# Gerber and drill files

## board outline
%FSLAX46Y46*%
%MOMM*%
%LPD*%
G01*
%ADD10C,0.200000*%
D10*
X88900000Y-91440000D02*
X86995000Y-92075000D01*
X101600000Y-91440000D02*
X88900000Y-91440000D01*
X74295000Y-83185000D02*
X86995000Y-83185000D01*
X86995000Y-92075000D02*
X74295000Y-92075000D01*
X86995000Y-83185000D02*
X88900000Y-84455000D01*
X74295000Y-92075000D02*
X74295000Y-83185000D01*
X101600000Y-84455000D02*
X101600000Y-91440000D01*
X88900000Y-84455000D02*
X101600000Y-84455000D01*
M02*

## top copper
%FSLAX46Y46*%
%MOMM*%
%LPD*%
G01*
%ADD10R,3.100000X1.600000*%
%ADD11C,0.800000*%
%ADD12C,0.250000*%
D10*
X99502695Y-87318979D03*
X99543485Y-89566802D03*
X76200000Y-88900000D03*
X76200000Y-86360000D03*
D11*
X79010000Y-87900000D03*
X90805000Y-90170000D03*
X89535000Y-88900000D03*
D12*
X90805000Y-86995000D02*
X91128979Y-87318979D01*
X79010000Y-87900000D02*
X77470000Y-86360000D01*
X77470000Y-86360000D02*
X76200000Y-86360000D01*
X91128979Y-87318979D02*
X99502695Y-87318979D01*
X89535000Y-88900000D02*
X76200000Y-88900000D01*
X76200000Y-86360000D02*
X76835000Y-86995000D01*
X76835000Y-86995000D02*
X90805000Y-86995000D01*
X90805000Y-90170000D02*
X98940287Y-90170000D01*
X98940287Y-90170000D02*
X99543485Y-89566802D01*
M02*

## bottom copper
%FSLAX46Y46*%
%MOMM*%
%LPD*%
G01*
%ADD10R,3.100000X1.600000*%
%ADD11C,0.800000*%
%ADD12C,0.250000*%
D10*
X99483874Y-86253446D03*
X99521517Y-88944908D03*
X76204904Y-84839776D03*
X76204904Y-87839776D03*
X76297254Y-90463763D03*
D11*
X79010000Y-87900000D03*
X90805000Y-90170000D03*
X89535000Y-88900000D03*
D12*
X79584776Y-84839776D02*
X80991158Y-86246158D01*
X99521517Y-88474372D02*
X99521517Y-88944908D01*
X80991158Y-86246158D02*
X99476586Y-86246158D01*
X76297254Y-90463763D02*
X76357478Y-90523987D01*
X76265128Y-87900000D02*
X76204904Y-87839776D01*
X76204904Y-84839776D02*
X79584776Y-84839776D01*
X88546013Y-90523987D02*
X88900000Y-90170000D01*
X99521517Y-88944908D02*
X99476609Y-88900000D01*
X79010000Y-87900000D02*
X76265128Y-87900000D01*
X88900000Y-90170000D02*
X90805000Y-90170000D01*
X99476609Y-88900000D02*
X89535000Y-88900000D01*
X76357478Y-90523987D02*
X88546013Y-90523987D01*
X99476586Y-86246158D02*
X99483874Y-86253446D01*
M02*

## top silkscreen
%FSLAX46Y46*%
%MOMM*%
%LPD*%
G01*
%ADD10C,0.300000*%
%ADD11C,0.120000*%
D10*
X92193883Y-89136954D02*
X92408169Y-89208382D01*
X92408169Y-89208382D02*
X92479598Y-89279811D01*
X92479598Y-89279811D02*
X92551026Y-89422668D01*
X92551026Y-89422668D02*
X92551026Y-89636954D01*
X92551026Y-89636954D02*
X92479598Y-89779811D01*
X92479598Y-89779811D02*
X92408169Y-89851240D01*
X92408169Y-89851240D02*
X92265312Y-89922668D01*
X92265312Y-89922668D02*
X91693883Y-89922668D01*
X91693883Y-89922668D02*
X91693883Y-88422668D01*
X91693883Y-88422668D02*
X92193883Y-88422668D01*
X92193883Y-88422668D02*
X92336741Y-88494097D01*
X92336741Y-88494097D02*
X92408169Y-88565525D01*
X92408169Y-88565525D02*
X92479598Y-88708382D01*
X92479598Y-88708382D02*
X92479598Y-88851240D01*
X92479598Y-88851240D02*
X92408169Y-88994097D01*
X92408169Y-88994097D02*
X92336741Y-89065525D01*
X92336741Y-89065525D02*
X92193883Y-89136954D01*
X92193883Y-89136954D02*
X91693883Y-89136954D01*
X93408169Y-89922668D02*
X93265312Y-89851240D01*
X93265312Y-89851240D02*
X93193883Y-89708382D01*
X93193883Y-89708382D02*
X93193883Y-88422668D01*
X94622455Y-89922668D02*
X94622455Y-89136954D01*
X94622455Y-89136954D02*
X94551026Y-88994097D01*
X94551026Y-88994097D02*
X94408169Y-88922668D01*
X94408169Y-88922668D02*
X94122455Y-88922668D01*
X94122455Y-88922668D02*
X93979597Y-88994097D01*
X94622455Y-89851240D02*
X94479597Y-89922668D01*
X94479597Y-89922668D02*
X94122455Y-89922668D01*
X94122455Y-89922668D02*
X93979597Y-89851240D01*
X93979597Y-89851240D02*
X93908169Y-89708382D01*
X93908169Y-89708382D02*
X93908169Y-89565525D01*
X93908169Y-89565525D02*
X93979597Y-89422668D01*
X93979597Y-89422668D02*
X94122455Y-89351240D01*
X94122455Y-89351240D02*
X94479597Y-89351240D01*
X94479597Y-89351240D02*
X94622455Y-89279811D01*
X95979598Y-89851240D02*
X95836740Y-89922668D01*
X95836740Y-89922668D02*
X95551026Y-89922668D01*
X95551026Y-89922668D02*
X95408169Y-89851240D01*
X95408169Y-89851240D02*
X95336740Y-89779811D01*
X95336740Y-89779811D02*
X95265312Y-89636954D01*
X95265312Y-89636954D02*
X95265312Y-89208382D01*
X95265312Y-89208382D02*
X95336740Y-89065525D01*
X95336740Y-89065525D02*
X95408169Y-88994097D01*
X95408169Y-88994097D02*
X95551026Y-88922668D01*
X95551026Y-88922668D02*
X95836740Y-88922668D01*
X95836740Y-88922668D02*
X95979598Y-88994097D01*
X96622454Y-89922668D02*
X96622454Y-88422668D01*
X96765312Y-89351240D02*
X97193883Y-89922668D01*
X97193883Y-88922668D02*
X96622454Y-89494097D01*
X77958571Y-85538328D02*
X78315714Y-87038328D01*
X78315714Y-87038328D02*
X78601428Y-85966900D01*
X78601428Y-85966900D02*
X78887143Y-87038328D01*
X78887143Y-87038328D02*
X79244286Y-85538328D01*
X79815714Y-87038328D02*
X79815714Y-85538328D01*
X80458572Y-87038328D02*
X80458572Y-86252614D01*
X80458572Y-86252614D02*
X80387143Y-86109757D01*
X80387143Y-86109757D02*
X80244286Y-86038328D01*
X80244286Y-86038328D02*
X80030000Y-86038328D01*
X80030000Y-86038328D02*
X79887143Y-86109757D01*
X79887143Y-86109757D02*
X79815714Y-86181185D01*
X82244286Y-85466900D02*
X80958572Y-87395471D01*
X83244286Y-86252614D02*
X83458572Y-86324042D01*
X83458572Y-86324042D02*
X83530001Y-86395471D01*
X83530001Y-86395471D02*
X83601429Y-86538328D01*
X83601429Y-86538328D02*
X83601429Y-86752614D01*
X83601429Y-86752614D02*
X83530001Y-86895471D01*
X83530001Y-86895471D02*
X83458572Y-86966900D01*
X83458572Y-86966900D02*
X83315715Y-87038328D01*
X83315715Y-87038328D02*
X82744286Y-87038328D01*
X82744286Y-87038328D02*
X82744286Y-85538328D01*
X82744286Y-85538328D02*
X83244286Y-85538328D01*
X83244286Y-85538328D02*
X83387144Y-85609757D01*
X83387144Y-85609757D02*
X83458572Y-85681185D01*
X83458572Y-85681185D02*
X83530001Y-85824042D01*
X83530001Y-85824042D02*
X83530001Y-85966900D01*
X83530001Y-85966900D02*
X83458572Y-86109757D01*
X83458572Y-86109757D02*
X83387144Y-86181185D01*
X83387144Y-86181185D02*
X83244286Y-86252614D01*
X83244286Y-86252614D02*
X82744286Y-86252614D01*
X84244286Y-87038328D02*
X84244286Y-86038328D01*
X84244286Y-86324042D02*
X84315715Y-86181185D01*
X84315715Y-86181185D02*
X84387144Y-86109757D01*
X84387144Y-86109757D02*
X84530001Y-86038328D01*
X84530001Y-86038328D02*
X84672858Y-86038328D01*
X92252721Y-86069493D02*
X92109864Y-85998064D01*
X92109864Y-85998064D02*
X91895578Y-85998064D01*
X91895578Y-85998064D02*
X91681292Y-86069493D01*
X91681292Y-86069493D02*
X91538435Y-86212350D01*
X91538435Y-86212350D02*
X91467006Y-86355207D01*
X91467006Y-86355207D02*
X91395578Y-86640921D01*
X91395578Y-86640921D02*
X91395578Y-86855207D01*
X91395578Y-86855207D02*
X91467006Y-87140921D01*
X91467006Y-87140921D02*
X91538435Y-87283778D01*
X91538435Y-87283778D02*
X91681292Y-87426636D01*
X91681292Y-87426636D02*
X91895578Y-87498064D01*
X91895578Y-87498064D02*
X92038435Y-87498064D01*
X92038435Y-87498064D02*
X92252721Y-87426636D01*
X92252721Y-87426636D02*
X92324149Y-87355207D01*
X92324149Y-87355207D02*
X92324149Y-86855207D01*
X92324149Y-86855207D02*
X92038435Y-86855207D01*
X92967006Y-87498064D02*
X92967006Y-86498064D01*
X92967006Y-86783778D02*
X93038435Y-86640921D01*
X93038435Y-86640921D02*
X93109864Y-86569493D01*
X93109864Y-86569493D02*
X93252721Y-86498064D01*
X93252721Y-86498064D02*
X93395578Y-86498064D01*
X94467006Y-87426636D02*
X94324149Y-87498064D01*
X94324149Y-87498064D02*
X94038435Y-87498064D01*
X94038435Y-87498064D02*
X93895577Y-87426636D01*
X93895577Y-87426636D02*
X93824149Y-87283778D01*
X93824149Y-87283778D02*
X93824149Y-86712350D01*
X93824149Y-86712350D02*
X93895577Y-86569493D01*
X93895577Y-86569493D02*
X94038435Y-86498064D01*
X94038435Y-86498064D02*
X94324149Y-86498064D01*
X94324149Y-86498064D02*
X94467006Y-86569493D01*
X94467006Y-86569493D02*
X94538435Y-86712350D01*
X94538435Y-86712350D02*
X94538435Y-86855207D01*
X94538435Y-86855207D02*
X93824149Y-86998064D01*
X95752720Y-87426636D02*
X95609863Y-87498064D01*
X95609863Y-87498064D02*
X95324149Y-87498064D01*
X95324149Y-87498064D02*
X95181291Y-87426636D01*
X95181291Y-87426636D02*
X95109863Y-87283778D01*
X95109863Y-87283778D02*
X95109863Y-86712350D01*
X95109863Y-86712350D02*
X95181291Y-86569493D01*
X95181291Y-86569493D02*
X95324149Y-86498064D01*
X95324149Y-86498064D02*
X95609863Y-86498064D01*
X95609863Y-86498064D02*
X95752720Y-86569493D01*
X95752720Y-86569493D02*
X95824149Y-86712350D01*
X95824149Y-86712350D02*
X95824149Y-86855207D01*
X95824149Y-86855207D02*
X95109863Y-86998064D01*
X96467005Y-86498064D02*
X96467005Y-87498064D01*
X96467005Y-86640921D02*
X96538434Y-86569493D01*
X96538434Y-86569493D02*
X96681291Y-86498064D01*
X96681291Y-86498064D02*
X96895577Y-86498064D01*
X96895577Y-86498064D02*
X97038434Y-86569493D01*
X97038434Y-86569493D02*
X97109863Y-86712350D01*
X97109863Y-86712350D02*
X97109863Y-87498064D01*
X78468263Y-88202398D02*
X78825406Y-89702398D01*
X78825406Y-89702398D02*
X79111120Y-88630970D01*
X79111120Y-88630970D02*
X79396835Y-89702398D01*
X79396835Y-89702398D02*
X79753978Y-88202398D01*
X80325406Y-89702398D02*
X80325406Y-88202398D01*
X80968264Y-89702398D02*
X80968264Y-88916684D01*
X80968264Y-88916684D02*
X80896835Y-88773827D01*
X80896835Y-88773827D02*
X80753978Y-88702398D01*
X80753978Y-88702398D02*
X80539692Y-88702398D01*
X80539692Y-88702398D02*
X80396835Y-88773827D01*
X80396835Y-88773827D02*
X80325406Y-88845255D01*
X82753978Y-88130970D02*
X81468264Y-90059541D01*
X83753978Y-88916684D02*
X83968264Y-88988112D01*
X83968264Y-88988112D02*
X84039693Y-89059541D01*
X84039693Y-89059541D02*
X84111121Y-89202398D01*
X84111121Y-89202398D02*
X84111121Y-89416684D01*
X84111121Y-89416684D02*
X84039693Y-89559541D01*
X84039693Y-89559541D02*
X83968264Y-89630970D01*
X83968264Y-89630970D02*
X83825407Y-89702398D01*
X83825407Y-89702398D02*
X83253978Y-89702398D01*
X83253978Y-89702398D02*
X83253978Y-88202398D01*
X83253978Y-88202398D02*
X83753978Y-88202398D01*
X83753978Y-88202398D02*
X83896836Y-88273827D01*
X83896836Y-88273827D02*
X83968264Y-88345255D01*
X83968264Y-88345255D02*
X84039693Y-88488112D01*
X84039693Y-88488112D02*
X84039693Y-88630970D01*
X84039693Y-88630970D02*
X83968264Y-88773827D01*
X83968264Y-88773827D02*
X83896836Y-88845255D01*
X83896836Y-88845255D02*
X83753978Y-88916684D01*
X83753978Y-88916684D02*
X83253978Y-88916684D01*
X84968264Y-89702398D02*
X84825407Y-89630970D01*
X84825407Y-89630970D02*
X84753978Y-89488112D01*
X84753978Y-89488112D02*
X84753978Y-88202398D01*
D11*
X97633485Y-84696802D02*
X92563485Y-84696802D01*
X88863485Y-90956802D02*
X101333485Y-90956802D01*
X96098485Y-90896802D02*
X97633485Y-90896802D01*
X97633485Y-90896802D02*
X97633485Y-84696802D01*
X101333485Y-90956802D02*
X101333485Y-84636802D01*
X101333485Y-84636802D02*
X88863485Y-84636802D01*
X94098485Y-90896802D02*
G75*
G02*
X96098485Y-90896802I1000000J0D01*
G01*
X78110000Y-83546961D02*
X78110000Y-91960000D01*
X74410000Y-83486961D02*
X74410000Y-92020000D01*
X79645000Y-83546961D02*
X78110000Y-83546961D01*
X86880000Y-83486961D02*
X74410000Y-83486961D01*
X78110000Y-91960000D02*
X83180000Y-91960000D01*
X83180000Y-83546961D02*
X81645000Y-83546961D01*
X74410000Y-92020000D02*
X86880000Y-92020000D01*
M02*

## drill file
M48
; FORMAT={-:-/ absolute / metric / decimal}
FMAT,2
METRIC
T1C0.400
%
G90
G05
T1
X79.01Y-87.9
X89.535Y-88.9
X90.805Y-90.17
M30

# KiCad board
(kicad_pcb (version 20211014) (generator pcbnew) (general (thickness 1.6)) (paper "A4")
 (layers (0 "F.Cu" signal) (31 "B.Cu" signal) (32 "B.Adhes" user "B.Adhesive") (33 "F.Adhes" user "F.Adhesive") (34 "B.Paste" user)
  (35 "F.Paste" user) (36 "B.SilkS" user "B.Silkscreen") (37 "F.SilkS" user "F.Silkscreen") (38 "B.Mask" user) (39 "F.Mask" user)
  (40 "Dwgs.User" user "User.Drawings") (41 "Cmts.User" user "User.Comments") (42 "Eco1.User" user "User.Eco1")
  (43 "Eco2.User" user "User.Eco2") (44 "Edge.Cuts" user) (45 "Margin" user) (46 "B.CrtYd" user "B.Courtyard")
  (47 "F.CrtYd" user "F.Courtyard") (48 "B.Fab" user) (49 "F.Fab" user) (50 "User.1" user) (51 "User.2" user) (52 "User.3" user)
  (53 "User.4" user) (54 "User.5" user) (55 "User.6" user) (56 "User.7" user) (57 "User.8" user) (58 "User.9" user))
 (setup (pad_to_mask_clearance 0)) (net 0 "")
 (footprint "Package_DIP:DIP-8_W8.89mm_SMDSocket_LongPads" (layer "F.Cu") (at 95.098485 85.756802 180)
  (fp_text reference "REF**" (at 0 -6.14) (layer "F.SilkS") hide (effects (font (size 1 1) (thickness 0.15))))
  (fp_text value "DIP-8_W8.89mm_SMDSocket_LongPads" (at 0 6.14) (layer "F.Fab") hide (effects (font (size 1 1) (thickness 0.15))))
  (fp_line (start -2.535 1.06) (end 2.535 1.06) (layer "F.SilkS") (width 0.12))
  (fp_line (start 6.235 -5.2) (end -6.235 -5.2) (layer "F.SilkS") (width 0.12))
  (fp_line (start -1 -5.14) (end -2.535 -5.14) (layer "F.SilkS") (width 0.12))
  (fp_line (start -2.535 -5.14) (end -2.535 1.06) (layer "F.SilkS") (width 0.12))
  (fp_line (start -6.235 -5.2) (end -6.235 1.12) (layer "F.SilkS") (width 0.12))
  (fp_line (start -6.235 1.12) (end 6.235 1.12) (layer "F.SilkS") (width 0.12))
  (fp_arc (start 1 -5.14) (mid 0 -4.14) (end -1 -5.14) (layer "F.SilkS") (width 0.12))
  (pad "GND" smd rect (at -4.385389 -0.496644 180) (size 3.1 1.6) (layers "B.Cu" "B.Paste" "B.Mask"))
  (pad "RX" smd rect (at -4.423032 -3.188106 180) (size 3.1 1.6) (layers "B.Cu" "B.Paste" "B.Mask"))
  (pad "TS" smd rect (at -4.40421 -1.562177 180) (size 3.1 1.6) (layers "F.Cu" "F.Paste" "F.Mask"))
  (pad "TX" smd rect (at -4.445 -3.81 180) (size 3.1 1.6) (layers "F.Cu" "F.Paste" "F.Mask")))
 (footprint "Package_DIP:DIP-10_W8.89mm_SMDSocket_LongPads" (layer "F.Cu") (at 80.645 88.9)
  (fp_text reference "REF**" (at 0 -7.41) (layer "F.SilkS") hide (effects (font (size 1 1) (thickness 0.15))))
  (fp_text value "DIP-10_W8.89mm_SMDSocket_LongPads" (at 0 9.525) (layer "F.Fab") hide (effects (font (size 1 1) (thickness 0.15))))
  (fp_line (start -2.535 -5.353039) (end -2.535 3.06) (layer "F.SilkS") (width 0.12))
  (fp_line (start -6.235 -5.413039) (end -6.235 3.12) (layer "F.SilkS") (width 0.12))
  (fp_line (start -1 -5.353039) (end -2.535 -5.353039) (layer "F.SilkS") (width 0.12))
  (fp_line (start 6.235 -5.413039) (end -6.235 -5.413039) (layer "F.SilkS") (width 0.12))
  (fp_line (start -2.535 3.06) (end 2.535 3.06) (layer "F.SilkS") (width 0.12))
  (fp_line (start 2.535 -5.353039) (end 1 -5.353039) (layer "F.SilkS") (width 0.12))
  (fp_line (start -6.235 3.12) (end 6.235 3.12) (layer "F.SilkS") (width 0.12))
  (pad "GND" smd rect (at -4.440096 -4.060224) (size 3.1 1.6) (layers "B.Cu" "B.Paste" "B.Mask"))
  (pad "RX" smd rect (at -4.445 0) (size 3.1 1.6) (layers "F.Cu" "F.Paste" "F.Mask"))
  (pad "TS" smd rect (at -4.440096 -1.060224) (size 3.1 1.6) (layers "B.Cu" "B.Paste" "B.Mask"))
  (pad "TS" smd rect (at -4.445 -2.54) (size 3.1 1.6) (layers "F.Cu" "F.Paste" "F.Mask"))
  (pad "TX" smd rect (at -4.347746 1.563763) (size 3.1 1.6) (layers "B.Cu" "B.Paste" "B.Mask")))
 (gr_line (start 88.9 91.44) (end 86.995 92.075) (layer "Edge.Cuts") (width 0.2))
 (gr_line (start 101.6 91.44) (end 88.9 91.44) (layer "Edge.Cuts") (width 0.2))
 (gr_line (start 74.295 83.185) (end 86.995 83.185) (layer "Edge.Cuts") (width 0.2))
 (gr_line (start 86.995 92.075) (end 74.295 92.075) (layer "Edge.Cuts") (width 0.2))
 (gr_line (start 86.995 83.185) (end 88.9 84.455) (layer "Edge.Cuts") (width 0.2))
 (gr_line (start 74.295 92.075) (end 74.295 83.185) (layer "Edge.Cuts") (width 0.2))
 (gr_line (start 101.6 84.455) (end 101.6 91.44) (layer "Edge.Cuts") (width 0.2))
 (gr_line (start 88.9 84.455) (end 101.6 84.455) (layer "Edge.Cuts") (width 0.2))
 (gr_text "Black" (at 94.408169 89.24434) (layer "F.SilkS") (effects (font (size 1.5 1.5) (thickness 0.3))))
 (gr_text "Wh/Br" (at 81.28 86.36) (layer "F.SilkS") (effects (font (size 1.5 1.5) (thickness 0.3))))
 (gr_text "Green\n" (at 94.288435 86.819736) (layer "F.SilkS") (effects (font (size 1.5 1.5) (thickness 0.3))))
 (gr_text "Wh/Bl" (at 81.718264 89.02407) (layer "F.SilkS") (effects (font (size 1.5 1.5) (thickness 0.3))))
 (segment (start 90.805 86.995) (end 91.128979 87.318979) (width 0.25) (layer "F.Cu") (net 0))
 (segment (start 79.01 87.9) (end 77.47 86.36) (width 0.25) (layer "F.Cu") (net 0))
 (segment (start 77.47 86.36) (end 76.2 86.36) (width 0.25) (layer "F.Cu") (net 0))
 (segment (start 91.128979 87.318979) (end 99.502695 87.318979) (width 0.25) (layer "F.Cu") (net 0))
 (segment (start 89.535 88.9) (end 76.2 88.9) (width 0.25) (layer "F.Cu") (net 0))
 (segment (start 76.2 86.36) (end 76.835 86.995) (width 0.25) (layer "F.Cu") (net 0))
 (segment (start 76.835 86.995) (end 90.805 86.995) (width 0.25) (layer "F.Cu") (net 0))
 (segment (start 90.805 90.17) (end 98.940287 90.17) (width 0.25) (layer "F.Cu") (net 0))
 (segment (start 98.940287 90.17) (end 99.543485 89.566802) (width 0.25) (layer "F.Cu") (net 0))
 (via (at 79.01 87.9) (size 0.8) (drill 0.4) (layers "F.Cu" "B.Cu") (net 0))
 (via (at 90.805 90.17) (size 0.8) (drill 0.4) (layers "F.Cu" "B.Cu") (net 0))
 (via (at 89.535 88.9) (size 0.8) (drill 0.4) (layers "F.Cu" "B.Cu") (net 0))
 (segment (start 79.584776 84.839776) (end 80.991158 86.246158) (width 0.25) (layer "B.Cu") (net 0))
 (segment (start 99.521517 88.474372) (end 99.521517 88.944908) (width 0.25) (layer "B.Cu") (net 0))
 (segment (start 80.991158 86.246158) (end 99.476586 86.246158) (width 0.25) (layer "B.Cu") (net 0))
 (segment (start 76.297254 90.463763) (end 76.357478 90.523987) (width 0.25) (layer "B.Cu") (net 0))
 (segment (start 76.265128 87.9) (end 76.204904 87.839776) (width 0.25) (layer "B.Cu") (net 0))
 (segment (start 76.204904 84.839776) (end 79.584776 84.839776) (width 0.25) (layer "B.Cu") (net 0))
 (segment (start 88.546013 90.523987) (end 88.9 90.17) (width 0.25) (layer "B.Cu") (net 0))
 (segment (start 99.521517 88.944908) (end 99.476609 88.9) (width 0.25) (layer "B.Cu") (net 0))
 (segment (start 79.01 87.9) (end 76.265128 87.9) (width 0.25) (layer "B.Cu") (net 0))
 (segment (start 88.9 90.17) (end 90.805 90.17) (width 0.25) (layer "B.Cu") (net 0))
 (segment (start 99.476609 88.9) (end 89.535 88.9) (width 0.25) (layer "B.Cu") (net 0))
 (segment (start 76.357478 90.523987) (end 88.546013 90.523987) (width 0.25) (layer "B.Cu") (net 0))
 (segment (start 99.476586 86.246158) (end 99.483874 86.253446) (width 0.25) (layer "B.Cu") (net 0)))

